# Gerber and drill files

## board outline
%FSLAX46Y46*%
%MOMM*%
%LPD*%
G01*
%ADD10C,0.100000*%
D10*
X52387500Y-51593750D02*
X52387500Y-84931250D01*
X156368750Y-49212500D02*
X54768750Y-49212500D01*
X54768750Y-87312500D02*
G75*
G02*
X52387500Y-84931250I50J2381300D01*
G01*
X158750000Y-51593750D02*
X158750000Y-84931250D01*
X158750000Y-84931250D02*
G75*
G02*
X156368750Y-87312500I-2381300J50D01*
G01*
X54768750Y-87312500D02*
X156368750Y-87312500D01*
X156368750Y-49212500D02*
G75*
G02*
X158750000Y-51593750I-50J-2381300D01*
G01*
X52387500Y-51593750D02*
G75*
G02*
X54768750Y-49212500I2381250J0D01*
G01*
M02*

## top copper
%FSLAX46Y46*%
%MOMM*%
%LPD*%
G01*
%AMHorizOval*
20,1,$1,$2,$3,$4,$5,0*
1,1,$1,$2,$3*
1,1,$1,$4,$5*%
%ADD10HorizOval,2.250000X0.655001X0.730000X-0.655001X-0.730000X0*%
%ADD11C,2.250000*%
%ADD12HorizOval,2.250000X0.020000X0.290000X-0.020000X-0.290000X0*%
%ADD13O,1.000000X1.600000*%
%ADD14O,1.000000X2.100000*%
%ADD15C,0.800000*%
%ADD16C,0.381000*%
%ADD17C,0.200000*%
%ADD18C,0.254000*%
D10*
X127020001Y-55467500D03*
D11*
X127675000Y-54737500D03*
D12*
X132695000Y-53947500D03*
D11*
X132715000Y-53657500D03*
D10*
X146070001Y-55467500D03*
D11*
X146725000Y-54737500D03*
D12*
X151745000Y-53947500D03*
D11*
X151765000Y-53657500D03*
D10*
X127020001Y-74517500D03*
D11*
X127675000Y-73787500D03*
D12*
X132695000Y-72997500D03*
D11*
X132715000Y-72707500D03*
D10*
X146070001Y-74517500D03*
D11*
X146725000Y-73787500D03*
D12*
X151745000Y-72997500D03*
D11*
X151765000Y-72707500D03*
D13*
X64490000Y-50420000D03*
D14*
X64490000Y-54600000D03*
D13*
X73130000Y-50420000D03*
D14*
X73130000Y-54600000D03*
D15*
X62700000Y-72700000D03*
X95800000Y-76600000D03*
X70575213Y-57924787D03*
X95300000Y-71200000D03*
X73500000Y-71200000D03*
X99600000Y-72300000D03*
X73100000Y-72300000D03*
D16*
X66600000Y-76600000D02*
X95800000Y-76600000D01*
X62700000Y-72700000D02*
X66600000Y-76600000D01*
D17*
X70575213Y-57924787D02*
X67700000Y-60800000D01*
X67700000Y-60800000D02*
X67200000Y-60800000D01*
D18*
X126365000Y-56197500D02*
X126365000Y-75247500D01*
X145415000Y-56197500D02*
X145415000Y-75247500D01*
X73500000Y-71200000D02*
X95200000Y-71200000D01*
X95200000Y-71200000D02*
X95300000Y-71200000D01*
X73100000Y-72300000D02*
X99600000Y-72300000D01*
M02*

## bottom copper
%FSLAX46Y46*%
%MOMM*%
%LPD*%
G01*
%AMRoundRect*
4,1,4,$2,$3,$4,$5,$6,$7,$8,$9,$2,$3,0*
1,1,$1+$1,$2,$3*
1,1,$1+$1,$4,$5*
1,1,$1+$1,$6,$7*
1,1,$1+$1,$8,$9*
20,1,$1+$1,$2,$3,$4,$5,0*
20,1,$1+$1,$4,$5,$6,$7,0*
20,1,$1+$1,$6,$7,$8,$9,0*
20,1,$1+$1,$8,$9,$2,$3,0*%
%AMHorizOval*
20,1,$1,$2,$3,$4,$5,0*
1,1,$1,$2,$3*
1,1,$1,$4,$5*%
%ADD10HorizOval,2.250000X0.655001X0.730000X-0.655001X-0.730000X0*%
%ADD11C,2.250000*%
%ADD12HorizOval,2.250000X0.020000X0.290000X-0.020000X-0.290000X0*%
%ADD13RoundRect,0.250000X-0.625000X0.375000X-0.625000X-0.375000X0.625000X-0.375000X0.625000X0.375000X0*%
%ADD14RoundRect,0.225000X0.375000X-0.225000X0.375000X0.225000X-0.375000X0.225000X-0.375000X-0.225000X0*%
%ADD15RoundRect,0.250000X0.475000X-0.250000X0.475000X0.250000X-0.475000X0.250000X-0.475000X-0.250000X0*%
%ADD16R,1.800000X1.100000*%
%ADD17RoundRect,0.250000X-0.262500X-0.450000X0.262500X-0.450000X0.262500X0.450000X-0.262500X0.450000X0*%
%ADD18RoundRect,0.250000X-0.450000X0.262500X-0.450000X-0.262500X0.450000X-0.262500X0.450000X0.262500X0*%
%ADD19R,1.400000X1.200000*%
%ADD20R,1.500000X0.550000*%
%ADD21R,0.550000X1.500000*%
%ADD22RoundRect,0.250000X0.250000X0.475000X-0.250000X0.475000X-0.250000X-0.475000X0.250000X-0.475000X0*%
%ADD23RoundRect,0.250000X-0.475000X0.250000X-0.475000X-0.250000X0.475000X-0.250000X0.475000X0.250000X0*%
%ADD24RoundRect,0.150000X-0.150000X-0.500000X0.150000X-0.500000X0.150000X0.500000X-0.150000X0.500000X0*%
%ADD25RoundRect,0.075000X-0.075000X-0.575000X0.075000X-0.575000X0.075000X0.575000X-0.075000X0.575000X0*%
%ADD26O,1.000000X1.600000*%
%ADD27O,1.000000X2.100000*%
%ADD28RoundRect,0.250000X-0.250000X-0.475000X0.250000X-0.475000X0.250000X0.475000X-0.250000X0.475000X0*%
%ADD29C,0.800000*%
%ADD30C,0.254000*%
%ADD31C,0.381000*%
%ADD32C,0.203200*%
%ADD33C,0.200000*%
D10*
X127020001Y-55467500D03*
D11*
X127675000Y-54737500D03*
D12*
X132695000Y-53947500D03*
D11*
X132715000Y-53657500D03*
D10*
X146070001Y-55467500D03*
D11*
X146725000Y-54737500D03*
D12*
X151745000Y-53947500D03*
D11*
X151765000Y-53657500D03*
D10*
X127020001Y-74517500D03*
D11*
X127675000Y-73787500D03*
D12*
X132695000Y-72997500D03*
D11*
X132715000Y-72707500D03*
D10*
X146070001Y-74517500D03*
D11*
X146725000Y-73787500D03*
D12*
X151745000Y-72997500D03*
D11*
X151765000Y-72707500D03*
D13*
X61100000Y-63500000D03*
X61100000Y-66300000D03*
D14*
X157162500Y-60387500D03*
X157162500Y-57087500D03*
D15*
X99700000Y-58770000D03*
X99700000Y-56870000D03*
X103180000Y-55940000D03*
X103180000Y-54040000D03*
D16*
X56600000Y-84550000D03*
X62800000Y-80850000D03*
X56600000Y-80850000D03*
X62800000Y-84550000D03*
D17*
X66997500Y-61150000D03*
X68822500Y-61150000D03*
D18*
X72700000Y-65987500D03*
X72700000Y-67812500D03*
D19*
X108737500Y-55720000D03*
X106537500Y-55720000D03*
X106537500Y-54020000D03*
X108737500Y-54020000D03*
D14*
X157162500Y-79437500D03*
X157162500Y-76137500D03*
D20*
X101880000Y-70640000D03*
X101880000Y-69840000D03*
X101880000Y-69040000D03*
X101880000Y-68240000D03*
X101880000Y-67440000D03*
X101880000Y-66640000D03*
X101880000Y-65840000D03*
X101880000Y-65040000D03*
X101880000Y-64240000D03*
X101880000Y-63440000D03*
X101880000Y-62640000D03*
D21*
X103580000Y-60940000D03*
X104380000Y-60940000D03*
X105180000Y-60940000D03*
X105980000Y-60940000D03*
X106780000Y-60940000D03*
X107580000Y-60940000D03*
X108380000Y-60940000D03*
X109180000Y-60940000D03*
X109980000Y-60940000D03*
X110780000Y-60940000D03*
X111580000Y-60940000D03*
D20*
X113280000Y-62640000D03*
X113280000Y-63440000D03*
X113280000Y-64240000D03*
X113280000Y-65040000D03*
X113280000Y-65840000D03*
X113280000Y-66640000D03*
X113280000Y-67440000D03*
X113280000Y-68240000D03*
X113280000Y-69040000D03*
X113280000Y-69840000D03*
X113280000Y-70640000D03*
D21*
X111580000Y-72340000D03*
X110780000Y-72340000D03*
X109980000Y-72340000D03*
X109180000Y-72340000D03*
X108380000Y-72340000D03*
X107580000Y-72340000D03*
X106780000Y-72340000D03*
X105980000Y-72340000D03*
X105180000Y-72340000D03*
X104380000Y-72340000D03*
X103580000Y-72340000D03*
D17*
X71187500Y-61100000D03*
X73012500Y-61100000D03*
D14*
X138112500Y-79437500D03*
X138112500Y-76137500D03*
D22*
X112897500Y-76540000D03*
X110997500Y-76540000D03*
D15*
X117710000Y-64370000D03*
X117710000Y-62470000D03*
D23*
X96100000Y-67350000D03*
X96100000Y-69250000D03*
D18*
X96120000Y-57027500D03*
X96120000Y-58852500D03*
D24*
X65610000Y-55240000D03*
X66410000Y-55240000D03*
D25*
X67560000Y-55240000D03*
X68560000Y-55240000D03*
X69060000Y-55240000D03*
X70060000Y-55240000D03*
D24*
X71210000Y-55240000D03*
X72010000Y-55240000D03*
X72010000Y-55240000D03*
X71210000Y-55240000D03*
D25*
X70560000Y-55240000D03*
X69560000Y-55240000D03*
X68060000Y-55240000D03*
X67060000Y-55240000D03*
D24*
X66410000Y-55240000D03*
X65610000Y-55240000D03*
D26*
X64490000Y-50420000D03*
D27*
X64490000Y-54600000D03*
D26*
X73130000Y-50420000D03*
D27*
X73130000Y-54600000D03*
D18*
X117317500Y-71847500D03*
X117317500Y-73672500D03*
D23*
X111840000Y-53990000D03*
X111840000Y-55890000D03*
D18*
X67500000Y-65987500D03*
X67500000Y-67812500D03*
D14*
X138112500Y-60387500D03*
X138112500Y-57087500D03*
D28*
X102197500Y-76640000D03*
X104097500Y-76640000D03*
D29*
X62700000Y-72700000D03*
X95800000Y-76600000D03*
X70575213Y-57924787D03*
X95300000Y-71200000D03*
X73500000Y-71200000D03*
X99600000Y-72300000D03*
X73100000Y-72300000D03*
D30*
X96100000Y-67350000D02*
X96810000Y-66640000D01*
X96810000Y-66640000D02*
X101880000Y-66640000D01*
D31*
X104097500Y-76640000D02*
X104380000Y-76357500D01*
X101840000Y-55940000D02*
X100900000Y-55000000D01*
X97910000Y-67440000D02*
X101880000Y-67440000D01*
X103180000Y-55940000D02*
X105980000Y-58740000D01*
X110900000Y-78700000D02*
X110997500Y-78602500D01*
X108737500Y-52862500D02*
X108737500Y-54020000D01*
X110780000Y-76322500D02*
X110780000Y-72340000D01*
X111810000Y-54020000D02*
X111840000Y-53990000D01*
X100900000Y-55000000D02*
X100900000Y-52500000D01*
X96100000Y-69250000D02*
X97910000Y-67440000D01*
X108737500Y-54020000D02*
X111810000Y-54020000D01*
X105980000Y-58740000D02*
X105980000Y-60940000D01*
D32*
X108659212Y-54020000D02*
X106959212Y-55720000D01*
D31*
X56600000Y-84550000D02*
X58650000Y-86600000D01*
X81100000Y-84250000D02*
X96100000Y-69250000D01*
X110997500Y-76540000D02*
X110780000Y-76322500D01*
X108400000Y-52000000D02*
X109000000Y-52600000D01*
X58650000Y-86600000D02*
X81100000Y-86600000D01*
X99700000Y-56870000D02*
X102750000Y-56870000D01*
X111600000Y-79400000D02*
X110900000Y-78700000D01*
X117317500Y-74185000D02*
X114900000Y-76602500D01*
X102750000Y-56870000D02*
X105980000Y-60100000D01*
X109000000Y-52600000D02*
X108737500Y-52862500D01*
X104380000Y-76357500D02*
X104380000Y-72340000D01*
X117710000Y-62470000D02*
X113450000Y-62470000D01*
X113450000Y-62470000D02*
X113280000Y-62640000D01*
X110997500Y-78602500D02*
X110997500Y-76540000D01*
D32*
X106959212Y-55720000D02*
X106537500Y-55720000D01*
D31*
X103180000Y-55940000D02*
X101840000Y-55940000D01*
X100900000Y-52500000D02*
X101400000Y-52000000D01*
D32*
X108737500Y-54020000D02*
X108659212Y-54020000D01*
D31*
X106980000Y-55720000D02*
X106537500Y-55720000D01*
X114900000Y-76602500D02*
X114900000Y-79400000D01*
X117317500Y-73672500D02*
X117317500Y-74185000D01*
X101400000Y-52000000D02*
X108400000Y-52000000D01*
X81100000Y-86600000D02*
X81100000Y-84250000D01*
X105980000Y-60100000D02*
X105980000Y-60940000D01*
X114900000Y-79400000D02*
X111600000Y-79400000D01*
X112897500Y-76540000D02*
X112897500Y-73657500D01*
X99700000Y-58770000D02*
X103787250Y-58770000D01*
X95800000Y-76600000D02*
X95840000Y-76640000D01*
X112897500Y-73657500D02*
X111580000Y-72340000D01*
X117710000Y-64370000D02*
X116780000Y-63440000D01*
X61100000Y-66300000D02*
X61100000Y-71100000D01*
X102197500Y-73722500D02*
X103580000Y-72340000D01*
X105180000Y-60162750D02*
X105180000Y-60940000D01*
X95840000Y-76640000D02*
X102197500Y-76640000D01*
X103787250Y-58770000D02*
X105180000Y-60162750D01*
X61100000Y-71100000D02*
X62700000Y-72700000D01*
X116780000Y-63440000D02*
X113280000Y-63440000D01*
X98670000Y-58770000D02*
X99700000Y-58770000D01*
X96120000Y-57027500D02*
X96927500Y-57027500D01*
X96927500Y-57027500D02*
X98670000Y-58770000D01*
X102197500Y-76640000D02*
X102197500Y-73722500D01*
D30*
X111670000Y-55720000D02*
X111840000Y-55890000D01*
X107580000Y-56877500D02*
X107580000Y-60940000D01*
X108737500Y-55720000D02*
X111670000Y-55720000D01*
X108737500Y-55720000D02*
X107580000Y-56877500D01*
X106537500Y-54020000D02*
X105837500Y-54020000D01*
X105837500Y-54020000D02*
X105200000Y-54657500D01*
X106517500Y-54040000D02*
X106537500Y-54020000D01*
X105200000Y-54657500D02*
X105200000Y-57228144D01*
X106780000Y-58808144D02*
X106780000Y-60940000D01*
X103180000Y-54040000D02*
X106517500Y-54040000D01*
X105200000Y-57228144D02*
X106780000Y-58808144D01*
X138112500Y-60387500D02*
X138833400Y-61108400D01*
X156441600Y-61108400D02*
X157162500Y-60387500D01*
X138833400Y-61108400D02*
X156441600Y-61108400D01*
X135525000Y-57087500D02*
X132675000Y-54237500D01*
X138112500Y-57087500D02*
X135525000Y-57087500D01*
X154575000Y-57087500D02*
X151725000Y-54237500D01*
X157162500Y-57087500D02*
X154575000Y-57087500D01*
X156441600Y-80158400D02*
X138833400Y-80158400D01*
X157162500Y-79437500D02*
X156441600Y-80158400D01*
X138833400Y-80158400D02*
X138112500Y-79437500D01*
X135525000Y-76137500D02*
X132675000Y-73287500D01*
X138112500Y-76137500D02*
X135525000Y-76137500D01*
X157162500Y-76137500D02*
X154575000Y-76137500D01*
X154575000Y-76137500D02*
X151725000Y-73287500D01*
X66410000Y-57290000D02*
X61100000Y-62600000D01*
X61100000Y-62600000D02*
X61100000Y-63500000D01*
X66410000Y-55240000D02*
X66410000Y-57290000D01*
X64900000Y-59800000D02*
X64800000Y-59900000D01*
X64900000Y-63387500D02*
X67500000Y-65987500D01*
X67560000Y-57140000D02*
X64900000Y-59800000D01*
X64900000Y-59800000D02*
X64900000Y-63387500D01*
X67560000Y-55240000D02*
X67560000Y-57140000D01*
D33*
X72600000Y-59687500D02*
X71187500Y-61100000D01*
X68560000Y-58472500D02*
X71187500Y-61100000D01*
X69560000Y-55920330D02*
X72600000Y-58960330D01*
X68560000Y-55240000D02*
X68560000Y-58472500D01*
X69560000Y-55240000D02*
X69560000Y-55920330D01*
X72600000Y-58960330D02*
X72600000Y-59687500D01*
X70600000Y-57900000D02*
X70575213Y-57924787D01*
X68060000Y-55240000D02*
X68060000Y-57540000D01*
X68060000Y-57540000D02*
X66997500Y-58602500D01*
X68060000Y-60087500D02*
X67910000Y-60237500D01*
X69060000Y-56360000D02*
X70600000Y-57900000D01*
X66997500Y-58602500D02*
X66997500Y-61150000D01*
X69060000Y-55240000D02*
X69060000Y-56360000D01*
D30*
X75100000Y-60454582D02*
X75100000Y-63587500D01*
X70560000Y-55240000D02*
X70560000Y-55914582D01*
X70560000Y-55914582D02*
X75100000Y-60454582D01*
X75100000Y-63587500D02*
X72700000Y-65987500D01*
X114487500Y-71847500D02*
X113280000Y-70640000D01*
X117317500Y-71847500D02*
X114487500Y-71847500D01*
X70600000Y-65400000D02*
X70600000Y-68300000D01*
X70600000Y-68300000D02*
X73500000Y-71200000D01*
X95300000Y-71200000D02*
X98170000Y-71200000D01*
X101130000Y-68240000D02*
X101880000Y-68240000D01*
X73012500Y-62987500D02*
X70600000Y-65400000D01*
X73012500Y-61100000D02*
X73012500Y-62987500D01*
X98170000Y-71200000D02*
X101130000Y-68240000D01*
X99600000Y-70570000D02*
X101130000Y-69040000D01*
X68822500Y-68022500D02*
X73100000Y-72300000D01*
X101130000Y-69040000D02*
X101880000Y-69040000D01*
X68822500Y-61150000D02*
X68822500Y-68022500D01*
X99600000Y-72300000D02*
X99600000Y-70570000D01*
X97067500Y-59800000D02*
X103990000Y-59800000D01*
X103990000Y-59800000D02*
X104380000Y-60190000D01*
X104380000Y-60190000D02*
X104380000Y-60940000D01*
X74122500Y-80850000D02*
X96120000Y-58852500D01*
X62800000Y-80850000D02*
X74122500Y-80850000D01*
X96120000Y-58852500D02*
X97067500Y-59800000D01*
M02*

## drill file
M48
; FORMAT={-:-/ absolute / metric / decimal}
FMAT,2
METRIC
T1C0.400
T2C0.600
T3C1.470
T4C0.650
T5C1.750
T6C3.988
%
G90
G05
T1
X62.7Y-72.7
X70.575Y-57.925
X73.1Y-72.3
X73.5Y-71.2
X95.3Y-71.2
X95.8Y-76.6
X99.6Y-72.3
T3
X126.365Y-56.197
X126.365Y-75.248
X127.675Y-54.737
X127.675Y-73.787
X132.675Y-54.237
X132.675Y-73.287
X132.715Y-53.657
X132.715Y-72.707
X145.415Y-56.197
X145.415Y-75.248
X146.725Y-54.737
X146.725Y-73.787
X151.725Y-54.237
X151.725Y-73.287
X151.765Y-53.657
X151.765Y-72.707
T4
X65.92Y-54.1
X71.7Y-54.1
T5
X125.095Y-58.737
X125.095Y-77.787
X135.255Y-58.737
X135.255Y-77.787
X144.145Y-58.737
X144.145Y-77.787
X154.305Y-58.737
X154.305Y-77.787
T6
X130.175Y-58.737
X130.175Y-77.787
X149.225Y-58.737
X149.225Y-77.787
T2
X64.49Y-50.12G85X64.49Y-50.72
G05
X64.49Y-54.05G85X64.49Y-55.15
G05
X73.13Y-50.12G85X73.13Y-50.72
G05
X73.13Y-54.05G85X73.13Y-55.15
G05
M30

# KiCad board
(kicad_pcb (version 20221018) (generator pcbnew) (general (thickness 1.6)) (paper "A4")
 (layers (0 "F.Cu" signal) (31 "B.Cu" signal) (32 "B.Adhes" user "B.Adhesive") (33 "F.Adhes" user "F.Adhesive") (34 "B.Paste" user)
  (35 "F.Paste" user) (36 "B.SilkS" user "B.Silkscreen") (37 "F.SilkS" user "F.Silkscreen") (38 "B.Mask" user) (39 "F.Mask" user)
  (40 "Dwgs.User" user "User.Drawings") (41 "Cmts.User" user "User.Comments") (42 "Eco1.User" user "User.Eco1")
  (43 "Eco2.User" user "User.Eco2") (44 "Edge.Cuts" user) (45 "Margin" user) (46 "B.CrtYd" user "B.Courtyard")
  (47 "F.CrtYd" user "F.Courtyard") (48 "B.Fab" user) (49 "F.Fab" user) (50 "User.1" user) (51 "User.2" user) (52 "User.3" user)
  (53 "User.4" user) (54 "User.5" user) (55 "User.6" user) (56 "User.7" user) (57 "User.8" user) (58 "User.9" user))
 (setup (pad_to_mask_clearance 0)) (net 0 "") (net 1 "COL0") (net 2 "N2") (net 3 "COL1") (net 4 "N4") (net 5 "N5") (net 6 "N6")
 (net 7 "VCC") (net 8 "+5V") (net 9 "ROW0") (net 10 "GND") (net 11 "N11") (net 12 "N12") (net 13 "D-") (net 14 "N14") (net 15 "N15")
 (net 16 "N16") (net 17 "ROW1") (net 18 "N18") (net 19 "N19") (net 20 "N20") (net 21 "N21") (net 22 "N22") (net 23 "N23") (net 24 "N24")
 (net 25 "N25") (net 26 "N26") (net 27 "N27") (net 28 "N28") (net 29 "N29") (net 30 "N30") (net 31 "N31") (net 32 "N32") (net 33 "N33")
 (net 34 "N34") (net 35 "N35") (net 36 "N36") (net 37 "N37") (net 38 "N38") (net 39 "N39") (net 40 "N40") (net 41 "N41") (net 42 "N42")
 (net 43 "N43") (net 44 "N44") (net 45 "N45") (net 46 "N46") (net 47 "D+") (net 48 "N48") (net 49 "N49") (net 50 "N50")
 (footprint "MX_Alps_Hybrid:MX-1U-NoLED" (layer "F.Cu") (at 130.175 58.7375)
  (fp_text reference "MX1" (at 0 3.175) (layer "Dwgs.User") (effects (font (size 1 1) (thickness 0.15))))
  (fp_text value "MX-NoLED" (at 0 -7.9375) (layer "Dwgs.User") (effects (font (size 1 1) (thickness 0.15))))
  (pad "" np_thru_hole circle (at -5.08 0 48.0996) (size 1.75 1.75) (drill 1.75) (layers "*.Cu" "*.Mask"))
  (pad "" np_thru_hole circle (at 0 0) (size 3.9878 3.9878) (drill 3.9878) (layers "*.Cu" "*.Mask"))
  (pad "" np_thru_hole circle (at 5.08 0 48.0996) (size 1.75 1.75) (drill 1.75) (layers "*.Cu" "*.Mask"))
  (pad "1" thru_hole oval (at -3.81 -2.54 48.0996) (size 4.211556 2.25) (drill 1.47 (offset 0.980778 0)) (layers "*.Cu" "B.Mask")
   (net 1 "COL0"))
  (pad "1" thru_hole circle (at -2.5 -4) (size 2.25 2.25) (drill 1.47) (layers "*.Cu" "B.Mask") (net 1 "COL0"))
  (pad "2" thru_hole oval (at 2.5 -4.5 86.0548) (size 2.831378 2.25) (drill 1.47 (offset 0.290689 0)) (layers "*.Cu" "B.Mask") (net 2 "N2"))
  (pad "2" thru_hole circle (at 2.54 -5.08) (size 2.25 2.25) (drill 1.47) (layers "*.Cu" "B.Mask") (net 2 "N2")))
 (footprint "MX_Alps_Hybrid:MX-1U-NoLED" (layer "F.Cu") (at 149.225 58.7375)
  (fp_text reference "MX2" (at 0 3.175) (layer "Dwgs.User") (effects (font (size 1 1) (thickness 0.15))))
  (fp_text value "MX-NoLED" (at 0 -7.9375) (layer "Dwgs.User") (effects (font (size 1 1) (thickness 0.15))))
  (pad "" np_thru_hole circle (at -5.08 0 48.0996) (size 1.75 1.75) (drill 1.75) (layers "*.Cu" "*.Mask"))
  (pad "" np_thru_hole circle (at 0 0) (size 3.9878 3.9878) (drill 3.9878) (layers "*.Cu" "*.Mask"))
  (pad "" np_thru_hole circle (at 5.08 0 48.0996) (size 1.75 1.75) (drill 1.75) (layers "*.Cu" "*.Mask"))
  (pad "1" thru_hole oval (at -3.81 -2.54 48.0996) (size 4.211556 2.25) (drill 1.47 (offset 0.980778 0)) (layers "*.Cu" "B.Mask")
   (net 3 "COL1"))
  (pad "1" thru_hole circle (at -2.5 -4) (size 2.25 2.25) (drill 1.47) (layers "*.Cu" "B.Mask") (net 3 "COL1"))
  (pad "2" thru_hole oval (at 2.5 -4.5 86.0548) (size 2.831378 2.25) (drill 1.47 (offset 0.290689 0)) (layers "*.Cu" "B.Mask") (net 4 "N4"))
  (pad "2" thru_hole circle (at 2.54 -5.08) (size 2.25 2.25) (drill 1.47) (layers "*.Cu" "B.Mask") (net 4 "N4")))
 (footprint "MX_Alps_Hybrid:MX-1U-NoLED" (layer "F.Cu") (at 130.175 77.7875)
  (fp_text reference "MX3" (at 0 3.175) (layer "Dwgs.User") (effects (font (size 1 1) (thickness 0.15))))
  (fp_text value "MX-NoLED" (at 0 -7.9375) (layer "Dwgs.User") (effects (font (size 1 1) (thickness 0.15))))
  (pad "" np_thru_hole circle (at -5.08 0 48.0996) (size 1.75 1.75) (drill 1.75) (layers "*.Cu" "*.Mask"))
  (pad "" np_thru_hole circle (at 0 0) (size 3.9878 3.9878) (drill 3.9878) (layers "*.Cu" "*.Mask"))
  (pad "" np_thru_hole circle (at 5.08 0 48.0996) (size 1.75 1.75) (drill 1.75) (layers "*.Cu" "*.Mask"))
  (pad "1" thru_hole oval (at -3.81 -2.54 48.0996) (size 4.211556 2.25) (drill 1.47 (offset 0.980778 0)) (layers "*.Cu" "B.Mask")
   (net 1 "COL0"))
  (pad "1" thru_hole circle (at -2.5 -4) (size 2.25 2.25) (drill 1.47) (layers "*.Cu" "B.Mask") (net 1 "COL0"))
  (pad "2" thru_hole oval (at 2.5 -4.5 86.0548) (size 2.831378 2.25) (drill 1.47 (offset 0.290689 0)) (layers "*.Cu" "B.Mask") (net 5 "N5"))
  (pad "2" thru_hole circle (at 2.54 -5.08) (size 2.25 2.25) (drill 1.47) (layers "*.Cu" "B.Mask") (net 5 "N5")))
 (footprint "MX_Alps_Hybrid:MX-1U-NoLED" (layer "F.Cu") (at 149.225 77.7875)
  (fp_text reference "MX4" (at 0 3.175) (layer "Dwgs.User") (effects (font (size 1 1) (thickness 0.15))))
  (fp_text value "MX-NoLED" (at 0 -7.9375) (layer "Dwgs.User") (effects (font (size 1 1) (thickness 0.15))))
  (pad "" np_thru_hole circle (at -5.08 0 48.0996) (size 1.75 1.75) (drill 1.75) (layers "*.Cu" "*.Mask"))
  (pad "" np_thru_hole circle (at 0 0) (size 3.9878 3.9878) (drill 3.9878) (layers "*.Cu" "*.Mask"))
  (pad "" np_thru_hole circle (at 5.08 0 48.0996) (size 1.75 1.75) (drill 1.75) (layers "*.Cu" "*.Mask"))
  (pad "1" thru_hole oval (at -3.81 -2.54 48.0996) (size 4.211556 2.25) (drill 1.47 (offset 0.980778 0)) (layers "*.Cu" "B.Mask")
   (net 3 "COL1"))
  (pad "1" thru_hole circle (at -2.5 -4) (size 2.25 2.25) (drill 1.47) (layers "*.Cu" "B.Mask") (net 3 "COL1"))
  (pad "2" thru_hole oval (at 2.5 -4.5 86.0548) (size 2.831378 2.25) (drill 1.47 (offset 0.290689 0)) (layers "*.Cu" "B.Mask") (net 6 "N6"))
  (pad "2" thru_hole circle (at 2.54 -5.08) (size 2.25 2.25) (drill 1.47) (layers "*.Cu" "B.Mask") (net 6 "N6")))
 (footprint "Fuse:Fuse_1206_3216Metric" (layer "B.Cu") (at 61.1 64.9 -90)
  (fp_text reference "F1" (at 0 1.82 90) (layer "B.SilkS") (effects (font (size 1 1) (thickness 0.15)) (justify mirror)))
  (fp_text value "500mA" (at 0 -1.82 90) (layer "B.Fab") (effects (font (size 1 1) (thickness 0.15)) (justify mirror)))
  (pad "1" smd roundrect (at -1.4 0 270) (size 1.25 1.75) (layers "B.Cu" "B.Paste" "B.Mask") (roundrect_rratio 0.2) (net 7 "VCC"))
  (pad "2" smd roundrect (at 1.4 0 270) (size 1.25 1.75) (layers "B.Cu" "B.Paste" "B.Mask") (roundrect_rratio 0.2) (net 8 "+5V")))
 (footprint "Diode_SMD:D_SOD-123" (layer "B.Cu") (at 157.1625 58.7375 90)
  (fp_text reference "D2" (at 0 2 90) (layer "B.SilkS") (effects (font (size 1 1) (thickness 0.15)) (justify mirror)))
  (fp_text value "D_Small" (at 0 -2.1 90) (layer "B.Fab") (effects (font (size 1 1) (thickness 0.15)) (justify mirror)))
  (pad "1" smd roundrect (at -1.65 0 90) (size 0.9 1.2) (layers "B.Cu" "B.Paste" "B.Mask") (roundrect_rratio 0.25) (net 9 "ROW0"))
  (pad "2" smd roundrect (at 1.65 0 90) (size 0.9 1.2) (layers "B.Cu" "B.Paste" "B.Mask") (roundrect_rratio 0.25) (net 4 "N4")))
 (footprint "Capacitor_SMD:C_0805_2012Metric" (layer "B.Cu") (at 99.7 57.82 90)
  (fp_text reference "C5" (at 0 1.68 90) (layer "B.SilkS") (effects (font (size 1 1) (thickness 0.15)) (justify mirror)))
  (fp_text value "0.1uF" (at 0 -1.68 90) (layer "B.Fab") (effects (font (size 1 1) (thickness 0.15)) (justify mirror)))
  (pad "1" smd roundrect (at -0.95 0 90) (size 1 1.45) (layers "B.Cu" "B.Paste" "B.Mask") (roundrect_rratio 0.25) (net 8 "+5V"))
  (pad "2" smd roundrect (at 0.95 0 90) (size 1 1.45) (layers "B.Cu" "B.Paste" "B.Mask") (roundrect_rratio 0.25) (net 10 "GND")))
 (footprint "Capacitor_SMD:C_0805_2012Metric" (layer "B.Cu") (at 103.18 54.99 90)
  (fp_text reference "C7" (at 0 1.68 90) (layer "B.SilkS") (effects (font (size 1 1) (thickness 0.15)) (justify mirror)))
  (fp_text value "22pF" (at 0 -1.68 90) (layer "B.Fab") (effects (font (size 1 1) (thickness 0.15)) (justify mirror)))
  (pad "1" smd roundrect (at -0.95 0 90) (size 1 1.45) (layers "B.Cu" "B.Paste" "B.Mask") (roundrect_rratio 0.25) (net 10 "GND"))
  (pad "2" smd roundrect (at 0.95 0 90) (size 1 1.45) (layers "B.Cu" "B.Paste" "B.Mask") (roundrect_rratio 0.25) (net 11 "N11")))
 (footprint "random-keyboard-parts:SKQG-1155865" (layer "B.Cu") (at 59.7 82.7 180)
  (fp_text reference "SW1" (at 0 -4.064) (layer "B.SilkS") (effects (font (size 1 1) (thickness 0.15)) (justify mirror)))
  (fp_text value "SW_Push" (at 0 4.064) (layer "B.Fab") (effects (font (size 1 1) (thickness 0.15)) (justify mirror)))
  (pad "1" smd rect (at 3.1 -1.85 180) (size 1.8 1.1) (layers "B.Cu" "B.Paste" "B.Mask") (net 10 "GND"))
  (pad "2" smd rect (at -3.1 1.85 180) (size 1.8 1.1) (layers "B.Cu" "B.Paste" "B.Mask") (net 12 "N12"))
  (pad "3" smd rect (at 3.1 1.85 180) (size 1.8 1.1) (layers "B.Cu" "B.Paste" "B.Mask"))
  (pad "4" smd rect (at -3.1 -1.85 180) (size 1.8 1.1) (layers "B.Cu" "B.Paste" "B.Mask")))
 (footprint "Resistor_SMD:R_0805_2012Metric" (layer "B.Cu") (at 67.91 61.15)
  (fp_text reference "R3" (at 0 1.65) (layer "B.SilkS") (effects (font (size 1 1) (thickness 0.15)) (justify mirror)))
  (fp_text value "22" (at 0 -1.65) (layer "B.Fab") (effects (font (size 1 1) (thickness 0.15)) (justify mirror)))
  (pad "1" smd roundrect (at -0.9125 0) (size 1.025 1.4) (layers "B.Cu" "B.Paste" "B.Mask") (roundrect_rratio 0.243902) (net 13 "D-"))
  (pad "2" smd roundrect (at 0.9125 0) (size 1.025 1.4) (layers "B.Cu" "B.Paste" "B.Mask") (roundrect_rratio 0.243902) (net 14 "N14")))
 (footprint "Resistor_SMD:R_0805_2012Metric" (layer "B.Cu") (at 72.7 66.9 -90)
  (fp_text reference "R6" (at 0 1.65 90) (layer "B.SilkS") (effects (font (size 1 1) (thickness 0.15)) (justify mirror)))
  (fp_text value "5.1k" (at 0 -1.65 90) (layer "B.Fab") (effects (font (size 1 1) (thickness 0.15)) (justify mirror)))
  (pad "1" smd roundrect (at -0.9125 0 270) (size 1.025 1.4) (layers "B.Cu" "B.Paste" "B.Mask") (roundrect_rratio 0.243902) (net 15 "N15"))
  (pad "2" smd roundrect (at 0.9125 0 270) (size 1.025 1.4) (layers "B.Cu" "B.Paste" "B.Mask") (roundrect_rratio 0.243902) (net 10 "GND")))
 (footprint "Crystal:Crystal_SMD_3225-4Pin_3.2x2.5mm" (layer "B.Cu") (at 107.6375 54.87 180)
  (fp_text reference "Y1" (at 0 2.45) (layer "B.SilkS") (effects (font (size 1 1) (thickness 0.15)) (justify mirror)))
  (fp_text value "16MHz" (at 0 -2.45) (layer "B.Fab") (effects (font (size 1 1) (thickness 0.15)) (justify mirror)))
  (pad "1" smd rect (at -1.1 -0.85 180) (size 1.4 1.2) (layers "B.Cu" "B.Paste" "B.Mask") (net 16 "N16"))
  (pad "2" smd rect (at 1.1 -0.85 180) (size 1.4 1.2) (layers "B.Cu" "B.Paste" "B.Mask") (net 10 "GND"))
  (pad "3" smd rect (at 1.1 0.85 180) (size 1.4 1.2) (layers "B.Cu" "B.Paste" "B.Mask") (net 11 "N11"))
  (pad "4" smd rect (at -1.1 0.85 180) (size 1.4 1.2) (layers "B.Cu" "B.Paste" "B.Mask") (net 10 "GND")))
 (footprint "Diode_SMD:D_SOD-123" (layer "B.Cu") (at 157.1625 77.7875 90)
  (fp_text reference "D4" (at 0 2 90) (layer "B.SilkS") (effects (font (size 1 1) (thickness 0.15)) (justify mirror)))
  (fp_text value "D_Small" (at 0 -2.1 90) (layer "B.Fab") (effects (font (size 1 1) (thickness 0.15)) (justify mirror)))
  (pad "1" smd roundrect (at -1.65 0 90) (size 0.9 1.2) (layers "B.Cu" "B.Paste" "B.Mask") (roundrect_rratio 0.25) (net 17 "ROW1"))
  (pad "2" smd roundrect (at 1.65 0 90) (size 0.9 1.2) (layers "B.Cu" "B.Paste" "B.Mask") (roundrect_rratio 0.25) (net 6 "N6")))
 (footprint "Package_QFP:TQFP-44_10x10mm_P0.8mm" (layer "B.Cu") (at 107.58 66.64)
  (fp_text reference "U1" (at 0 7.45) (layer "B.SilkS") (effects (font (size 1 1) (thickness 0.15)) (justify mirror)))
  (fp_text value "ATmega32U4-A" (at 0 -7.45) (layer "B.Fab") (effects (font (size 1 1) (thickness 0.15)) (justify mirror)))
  (pad "1" smd rect (at -5.7 4) (size 1.5 0.55) (layers "B.Cu" "B.Paste" "B.Mask") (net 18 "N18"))
  (pad "2" smd rect (at -5.7 3.2) (size 1.5 0.55) (layers "B.Cu" "B.Paste" "B.Mask") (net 8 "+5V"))
  (pad "3" smd rect (at -5.7 2.4) (size 1.5 0.55) (layers "B.Cu" "B.Paste" "B.Mask") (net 14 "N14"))
  (pad "4" smd rect (at -5.7 1.6) (size 1.5 0.55) (layers "B.Cu" "B.Paste" "B.Mask") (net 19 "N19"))
  (pad "5" smd rect (at -5.7 0.8) (size 1.5 0.55) (layers "B.Cu" "B.Paste" "B.Mask") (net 10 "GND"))
  (pad "6" smd rect (at -5.7 0) (size 1.5 0.55) (layers "B.Cu" "B.Paste" "B.Mask") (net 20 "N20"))
  (pad "7" smd rect (at -5.7 -0.8) (size 1.5 0.55) (layers "B.Cu" "B.Paste" "B.Mask") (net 8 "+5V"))
  (pad "8" smd rect (at -5.7 -1.6) (size 1.5 0.55) (layers "B.Cu" "B.Paste" "B.Mask") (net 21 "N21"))
  (pad "9" smd rect (at -5.7 -2.4) (size 1.5 0.55) (layers "B.Cu" "B.Paste" "B.Mask") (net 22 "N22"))
  (pad "10" smd rect (at -5.7 -3.2) (size 1.5 0.55) (layers "B.Cu" "B.Paste" "B.Mask") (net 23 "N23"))
  (pad "11" smd rect (at -5.7 -4) (size 1.5 0.55) (layers "B.Cu" "B.Paste" "B.Mask") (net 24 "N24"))
  (pad "12" smd rect (at -4 -5.7 270) (size 1.5 0.55) (layers "B.Cu" "B.Paste" "B.Mask") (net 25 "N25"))
  (pad "13" smd rect (at -3.2 -5.7 270) (size 1.5 0.55) (layers "B.Cu" "B.Paste" "B.Mask") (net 12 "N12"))
  (pad "14" smd rect (at -2.4 -5.7 270) (size 1.5 0.55) (layers "B.Cu" "B.Paste" "B.Mask") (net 8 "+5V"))
  (pad "15" smd rect (at -1.6 -5.7 270) (size 1.5 0.55) (layers "B.Cu" "B.Paste" "B.Mask") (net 10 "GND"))
  (pad "16" smd rect (at -0.8 -5.7 270) (size 1.5 0.55) (layers "B.Cu" "B.Paste" "B.Mask") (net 11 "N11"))
  (pad "17" smd rect (at 0 -5.7 270) (size 1.5 0.55) (layers "B.Cu" "B.Paste" "B.Mask") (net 16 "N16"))
  (pad "18" smd rect (at 0.8 -5.7 270) (size 1.5 0.55) (layers "B.Cu" "B.Paste" "B.Mask") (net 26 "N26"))
  (pad "19" smd rect (at 1.6 -5.7 270) (size 1.5 0.55) (layers "B.Cu" "B.Paste" "B.Mask") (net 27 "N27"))
  (pad "20" smd rect (at 2.4 -5.7 270) (size 1.5 0.55) (layers "B.Cu" "B.Paste" "B.Mask") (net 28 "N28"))
  (pad "21" smd rect (at 3.2 -5.7 270) (size 1.5 0.55) (layers "B.Cu" "B.Paste" "B.Mask") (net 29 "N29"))
  (pad "22" smd rect (at 4 -5.7 270) (size 1.5 0.55) (layers "B.Cu" "B.Paste" "B.Mask") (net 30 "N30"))
  (pad "23" smd rect (at 5.7 -4) (size 1.5 0.55) (layers "B.Cu" "B.Paste" "B.Mask") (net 10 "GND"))
  (pad "24" smd rect (at 5.7 -3.2) (size 1.5 0.55) (layers "B.Cu" "B.Paste" "B.Mask") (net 8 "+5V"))
  (pad "25" smd rect (at 5.7 -2.4) (size 1.5 0.55) (layers "B.Cu" "B.Paste" "B.Mask") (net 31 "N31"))
  (pad "26" smd rect (at 5.7 -1.6) (size 1.5 0.55) (layers "B.Cu" "B.Paste" "B.Mask") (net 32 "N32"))
  (pad "27" smd rect (at 5.7 -0.8) (size 1.5 0.55) (layers "B.Cu" "B.Paste" "B.Mask") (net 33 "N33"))
  (pad "28" smd rect (at 5.7 0) (size 1.5 0.55) (layers "B.Cu" "B.Paste" "B.Mask") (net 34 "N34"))
  (pad "29" smd rect (at 5.7 0.8) (size 1.5 0.55) (layers "B.Cu" "B.Paste" "B.Mask") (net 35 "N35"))
  (pad "30" smd rect (at 5.7 1.6) (size 1.5 0.55) (layers "B.Cu" "B.Paste" "B.Mask") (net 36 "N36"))
  (pad "31" smd rect (at 5.7 2.4) (size 1.5 0.55) (layers "B.Cu" "B.Paste" "B.Mask") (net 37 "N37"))
  (pad "32" smd rect (at 5.7 3.2) (size 1.5 0.55) (layers "B.Cu" "B.Paste" "B.Mask") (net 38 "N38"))
  (pad "33" smd rect (at 5.7 4) (size 1.5 0.55) (layers "B.Cu" "B.Paste" "B.Mask") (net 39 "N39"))
  (pad "34" smd rect (at 4 5.7 270) (size 1.5 0.55) (layers "B.Cu" "B.Paste" "B.Mask") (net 8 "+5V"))
  (pad "35" smd rect (at 3.2 5.7 270) (size 1.5 0.55) (layers "B.Cu" "B.Paste" "B.Mask") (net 10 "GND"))
  (pad "36" smd rect (at 2.4 5.7 270) (size 1.5 0.55) (layers "B.Cu" "B.Paste" "B.Mask") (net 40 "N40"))
  (pad "37" smd rect (at 1.6 5.7 270) (size 1.5 0.55) (layers "B.Cu" "B.Paste" "B.Mask") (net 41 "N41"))
  (pad "38" smd rect (at 0.8 5.7 270) (size 1.5 0.55) (layers "B.Cu" "B.Paste" "B.Mask") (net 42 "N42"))
  (pad "39" smd rect (at 0 5.7 270) (size 1.5 0.55) (layers "B.Cu" "B.Paste" "B.Mask") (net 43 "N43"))
  (pad "40" smd rect (at -0.8 5.7 270) (size 1.5 0.55) (layers "B.Cu" "B.Paste" "B.Mask") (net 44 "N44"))
  (pad "41" smd rect (at -1.6 5.7 270) (size 1.5 0.55) (layers "B.Cu" "B.Paste" "B.Mask") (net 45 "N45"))
  (pad "42" smd rect (at -2.4 5.7 270) (size 1.5 0.55) (layers "B.Cu" "B.Paste" "B.Mask") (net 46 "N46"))
  (pad "43" smd rect (at -3.2 5.7 270) (size 1.5 0.55) (layers "B.Cu" "B.Paste" "B.Mask") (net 10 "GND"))
  (pad "44" smd rect (at -4 5.7 270) (size 1.5 0.55) (layers "B.Cu" "B.Paste" "B.Mask") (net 8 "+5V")))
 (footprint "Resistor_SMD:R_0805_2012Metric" (layer "B.Cu") (at 72.1 61.1)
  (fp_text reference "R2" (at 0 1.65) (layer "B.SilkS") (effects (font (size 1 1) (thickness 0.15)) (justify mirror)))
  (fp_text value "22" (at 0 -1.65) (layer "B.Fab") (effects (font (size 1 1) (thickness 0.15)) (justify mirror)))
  (pad "1" smd roundrect (at -0.9125 0) (size 1.025 1.4) (layers "B.Cu" "B.Paste" "B.Mask") (roundrect_rratio 0.243902) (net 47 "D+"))
  (pad "2" smd roundrect (at 0.9125 0) (size 1.025 1.4) (layers "B.Cu" "B.Paste" "B.Mask") (roundrect_rratio 0.243902) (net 19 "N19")))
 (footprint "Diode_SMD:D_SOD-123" (layer "B.Cu") (at 138.1125 77.7875 90)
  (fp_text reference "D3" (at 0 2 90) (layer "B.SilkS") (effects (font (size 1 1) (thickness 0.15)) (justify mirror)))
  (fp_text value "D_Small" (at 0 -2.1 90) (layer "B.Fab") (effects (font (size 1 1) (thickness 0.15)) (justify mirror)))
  (pad "1" smd roundrect (at -1.65 0 90) (size 0.9 1.2) (layers "B.Cu" "B.Paste" "B.Mask") (roundrect_rratio 0.25) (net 17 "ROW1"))
  (pad "2" smd roundrect (at 1.65 0 90) (size 0.9 1.2) (layers "B.Cu" "B.Paste" "B.Mask") (roundrect_rratio 0.25) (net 5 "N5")))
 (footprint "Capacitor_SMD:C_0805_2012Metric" (layer "B.Cu") (at 111.9475 76.54 180)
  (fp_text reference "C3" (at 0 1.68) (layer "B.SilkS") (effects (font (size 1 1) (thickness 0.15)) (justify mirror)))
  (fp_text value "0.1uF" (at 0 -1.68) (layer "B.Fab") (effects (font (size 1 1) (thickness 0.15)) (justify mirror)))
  (pad "1" smd roundrect (at -0.95 0 180) (size 1 1.45) (layers "B.Cu" "B.Paste" "B.Mask") (roundrect_rratio 0.25) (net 8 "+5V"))
  (pad "2" smd roundrect (at 0.95 0 180) (size 1 1.45) (layers "B.Cu" "B.Paste" "B.Mask") (roundrect_rratio 0.25) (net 10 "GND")))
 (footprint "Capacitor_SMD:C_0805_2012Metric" (layer "B.Cu") (at 117.71 63.42 90)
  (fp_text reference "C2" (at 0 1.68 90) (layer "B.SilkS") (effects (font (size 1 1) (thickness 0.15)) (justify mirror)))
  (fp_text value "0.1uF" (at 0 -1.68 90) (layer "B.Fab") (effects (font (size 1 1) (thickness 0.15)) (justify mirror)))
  (pad "1" smd roundrect (at -0.95 0 90) (size 1 1.45) (layers "B.Cu" "B.Paste" "B.Mask") (roundrect_rratio 0.25) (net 8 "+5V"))
  (pad "2" smd roundrect (at 0.95 0 90) (size 1 1.45) (layers "B.Cu" "B.Paste" "B.Mask") (roundrect_rratio 0.25) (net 10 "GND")))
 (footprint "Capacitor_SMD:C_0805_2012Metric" (layer "B.Cu") (at 96.1 68.3 -90)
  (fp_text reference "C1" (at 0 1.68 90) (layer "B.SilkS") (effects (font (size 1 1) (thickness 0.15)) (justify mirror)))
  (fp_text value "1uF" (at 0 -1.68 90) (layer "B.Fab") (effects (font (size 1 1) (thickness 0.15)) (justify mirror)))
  (pad "1" smd roundrect (at -0.95 0 270) (size 1 1.45) (layers "B.Cu" "B.Paste" "B.Mask") (roundrect_rratio 0.25) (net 20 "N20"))
  (pad "2" smd roundrect (at 0.95 0 270) (size 1 1.45) (layers "B.Cu" "B.Paste" "B.Mask") (roundrect_rratio 0.25) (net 10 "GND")))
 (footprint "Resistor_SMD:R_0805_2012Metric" (layer "B.Cu") (at 96.12 57.94 -90)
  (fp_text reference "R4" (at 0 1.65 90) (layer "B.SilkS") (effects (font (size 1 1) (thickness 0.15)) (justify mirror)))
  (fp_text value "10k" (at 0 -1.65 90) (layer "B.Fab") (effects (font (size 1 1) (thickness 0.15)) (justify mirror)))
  (pad "1" smd roundrect (at -0.9125 0 270) (size 1.025 1.4) (layers "B.Cu" "B.Paste" "B.Mask") (roundrect_rratio 0.243902) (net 8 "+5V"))
  (pad "2" smd roundrect (at 0.9125 0 270) (size 1.025 1.4) (layers "B.Cu" "B.Paste" "B.Mask") (roundrect_rratio 0.243902) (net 12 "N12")))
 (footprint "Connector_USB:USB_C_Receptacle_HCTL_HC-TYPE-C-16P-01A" (layer "B.Cu") (at 68.81 51.495)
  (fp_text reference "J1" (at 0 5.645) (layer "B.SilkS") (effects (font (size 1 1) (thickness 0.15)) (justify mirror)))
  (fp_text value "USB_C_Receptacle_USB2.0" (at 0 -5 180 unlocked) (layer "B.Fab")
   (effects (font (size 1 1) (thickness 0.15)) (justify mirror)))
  (pad "" np_thru_hole circle (at -2.89 2.605) (size 0.65 0.65) (drill 0.65) (layers "*.Mask"))
  (pad "" np_thru_hole circle (at 2.89 2.605) (size 0.65 0.65) (drill 0.65) (layers "*.Mask"))
  (pad "A1" smd roundrect (at -3.2 3.745) (size 0.6 1.3) (layers "B.Cu" "B.Paste" "B.Mask") (roundrect_rratio 0.25) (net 10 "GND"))
  (pad "A4" smd roundrect (at -2.4 3.745) (size 0.6 1.3) (layers "B.Cu" "B.Paste" "B.Mask") (roundrect_rratio 0.25) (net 7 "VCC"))
  (pad "A5" smd roundrect (at -1.25 3.745) (size 0.3 1.3) (layers "B.Cu" "B.Paste" "B.Mask") (roundrect_rratio 0.25) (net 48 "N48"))
  (pad "A6" smd roundrect (at -0.25 3.745) (size 0.3 1.3) (layers "B.Cu" "B.Paste" "B.Mask") (roundrect_rratio 0.25) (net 47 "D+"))
  (pad "A7" smd roundrect (at 0.25 3.745) (size 0.3 1.3) (layers "B.Cu" "B.Paste" "B.Mask") (roundrect_rratio 0.25) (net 13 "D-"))
  (pad "A8" smd roundrect (at 1.25 3.745) (size 0.3 1.3) (layers "B.Cu" "B.Paste" "B.Mask") (roundrect_rratio 0.25) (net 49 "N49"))
  (pad "A9" smd roundrect (at 2.4 3.745) (size 0.6 1.3) (layers "B.Cu" "B.Paste" "B.Mask") (roundrect_rratio 0.25) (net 7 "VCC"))
  (pad "A12" smd roundrect (at 3.2 3.745) (size 0.6 1.3) (layers "B.Cu" "B.Paste" "B.Mask") (roundrect_rratio 0.25) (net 10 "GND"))
  (pad "B1" smd roundrect (at 3.2 3.745) (size 0.6 1.3) (layers "B.Cu" "B.Paste" "B.Mask") (roundrect_rratio 0.25) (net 10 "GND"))
  (pad "B4" smd roundrect (at 2.4 3.745) (size 0.6 1.3) (layers "B.Cu" "B.Paste" "B.Mask") (roundrect_rratio 0.25) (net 7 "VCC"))
  (pad "B5" smd roundrect (at 1.75 3.745) (size 0.3 1.3) (layers "B.Cu" "B.Paste" "B.Mask") (roundrect_rratio 0.25) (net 15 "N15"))
  (pad "B6" smd roundrect (at 0.75 3.745) (size 0.3 1.3) (layers "B.Cu" "B.Paste" "B.Mask") (roundrect_rratio 0.25) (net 47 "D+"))
  (pad "B7" smd roundrect (at -0.75 3.745) (size 0.3 1.3) (layers "B.Cu" "B.Paste" "B.Mask") (roundrect_rratio 0.25) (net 13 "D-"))
  (pad "B8" smd roundrect (at -1.75 3.745) (size 0.3 1.3) (layers "B.Cu" "B.Paste" "B.Mask") (roundrect_rratio 0.25) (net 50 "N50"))
  (pad "B9" smd roundrect (at -2.4 3.745) (size 0.6 1.3) (layers "B.Cu" "B.Paste" "B.Mask") (roundrect_rratio 0.25) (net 7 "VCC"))
  (pad "B12" smd roundrect (at -3.2 3.745) (size 0.6 1.3) (layers "B.Cu" "B.Paste" "B.Mask") (roundrect_rratio 0.25) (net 10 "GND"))
  (pad "S1" thru_hole oval (at -4.32 -1.075) (size 1 1.6) (drill oval 0.6 1.2) (layers "*.Cu" "*.Mask") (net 10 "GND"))
  (pad "S1" thru_hole oval (at -4.32 3.105) (size 1 2.1) (drill oval 0.6 1.7) (layers "*.Cu" "*.Mask") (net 10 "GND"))
  (pad "S1" thru_hole oval (at 4.32 -1.075) (size 1 1.6) (drill oval 0.6 1.2) (layers "*.Cu" "*.Mask") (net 10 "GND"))
  (pad "S1" thru_hole oval (at 4.32 3.105) (size 1 2.1) (drill oval 0.6 1.7) (layers "*.Cu" "*.Mask") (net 10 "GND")))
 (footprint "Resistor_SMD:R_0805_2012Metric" (layer "B.Cu") (at 117.3175 72.76 -90)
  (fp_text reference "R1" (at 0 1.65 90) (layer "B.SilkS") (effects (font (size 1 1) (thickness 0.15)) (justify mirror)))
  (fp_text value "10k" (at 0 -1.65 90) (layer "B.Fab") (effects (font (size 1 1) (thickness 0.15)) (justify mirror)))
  (pad "1" smd roundrect (at -0.9125 0 270) (size 1.025 1.4) (layers "B.Cu" "B.Paste" "B.Mask") (roundrect_rratio 0.243902) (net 39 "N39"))
  (pad "2" smd roundrect (at 0.9125 0 270) (size 1.025 1.4) (layers "B.Cu" "B.Paste" "B.Mask") (roundrect_rratio 0.243902) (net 10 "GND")))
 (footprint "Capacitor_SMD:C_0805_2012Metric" (layer "B.Cu") (at 111.84 54.94 -90)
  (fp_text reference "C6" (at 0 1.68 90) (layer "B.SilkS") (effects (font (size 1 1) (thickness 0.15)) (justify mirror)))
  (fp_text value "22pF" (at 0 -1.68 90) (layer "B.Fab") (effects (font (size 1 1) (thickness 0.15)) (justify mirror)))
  (pad "1" smd roundrect (at -0.95 0 270) (size 1 1.45) (layers "B.Cu" "B.Paste" "B.Mask") (roundrect_rratio 0.25) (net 10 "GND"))
  (pad "2" smd roundrect (at 0.95 0 270) (size 1 1.45) (layers "B.Cu" "B.Paste" "B.Mask") (roundrect_rratio 0.25) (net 16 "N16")))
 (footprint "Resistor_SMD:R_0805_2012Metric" (layer "B.Cu") (at 67.5 66.9 -90)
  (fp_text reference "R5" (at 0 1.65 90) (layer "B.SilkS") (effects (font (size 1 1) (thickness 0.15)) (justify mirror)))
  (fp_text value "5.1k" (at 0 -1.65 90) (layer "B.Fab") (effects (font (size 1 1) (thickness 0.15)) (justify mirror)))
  (pad "1" smd roundrect (at -0.9125 0 270) (size 1.025 1.4) (layers "B.Cu" "B.Paste" "B.Mask") (roundrect_rratio 0.243902) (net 48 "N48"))
  (pad "2" smd roundrect (at 0.9125 0 270) (size 1.025 1.4) (layers "B.Cu" "B.Paste" "B.Mask") (roundrect_rratio 0.243902) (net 10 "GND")))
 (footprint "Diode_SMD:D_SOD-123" (layer "B.Cu") (at 138.1125 58.7375 90)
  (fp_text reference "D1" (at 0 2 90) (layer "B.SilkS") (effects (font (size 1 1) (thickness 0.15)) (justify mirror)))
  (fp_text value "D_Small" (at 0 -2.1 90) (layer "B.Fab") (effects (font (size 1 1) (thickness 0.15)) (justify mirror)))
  (pad "1" smd roundrect (at -1.65 0 90) (size 0.9 1.2) (layers "B.Cu" "B.Paste" "B.Mask") (roundrect_rratio 0.25) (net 9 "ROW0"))
  (pad "2" smd roundrect (at 1.65 0 90) (size 0.9 1.2) (layers "B.Cu" "B.Paste" "B.Mask") (roundrect_rratio 0.25) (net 2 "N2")))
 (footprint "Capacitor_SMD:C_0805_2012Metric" (layer "B.Cu") (at 103.1475 76.64)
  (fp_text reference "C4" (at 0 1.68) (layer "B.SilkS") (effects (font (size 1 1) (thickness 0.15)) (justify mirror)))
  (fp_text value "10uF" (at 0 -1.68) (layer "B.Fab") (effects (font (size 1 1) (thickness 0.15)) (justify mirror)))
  (pad "1" smd roundrect (at -0.95 0) (size 1 1.45) (layers "B.Cu" "B.Paste" "B.Mask") (roundrect_rratio 0.25) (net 8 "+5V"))
  (pad "2" smd roundrect (at 0.95 0) (size 1 1.45) (layers "B.Cu" "B.Paste" "B.Mask") (roundrect_rratio 0.25) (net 10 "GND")))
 (gr_line (start 52.3875 51.59375) (end 52.3875 84.93125) (stroke (width 0.1) (type default)) (layer "Edge.Cuts"))
 (gr_line (start 156.36875 49.2125) (end 54.76875 49.2125) (stroke (width 0.1) (type default)) (layer "Edge.Cuts"))
 (gr_arc (start 54.76875 87.3125) (mid 53.084952 86.615048) (end 52.3875 84.93125) (stroke (width 0.1) (type default)) (layer "Edge.Cuts"))
 (gr_line (start 158.75 51.59375) (end 158.75 84.93125) (stroke (width 0.1) (type default)) (layer "Edge.Cuts"))
 (gr_arc (start 158.75 84.93125) (mid 158.052548 86.615048) (end 156.36875 87.3125) (stroke (width 0.1) (type default)) (layer "Edge.Cuts"))
 (gr_line (start 54.76875 87.3125) (end 156.36875 87.3125) (stroke (width 0.1) (type default)) (layer "Edge.Cuts"))
 (gr_arc (start 156.36875 49.2125) (mid 158.052548 49.909952) (end 158.75 51.59375) (stroke (width 0.1) (type default)) (layer "Edge.Cuts"))
 (gr_arc (start 52.3875 51.59375) (mid 53.084952 49.909952) (end 54.76875 49.2125) (stroke (width 0.1) (type default)) (layer "Edge.Cuts"))
 (segment (start 96.1 67.35) (end 96.81 66.64) (width 0.254) (layer "B.Cu") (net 20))
 (segment (start 96.81 66.64) (end 101.88 66.64) (width 0.254) (layer "B.Cu") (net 20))
 (segment (start 104.0975 76.64) (end 104.38 76.3575) (width 0.381) (layer "B.Cu") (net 10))
 (segment (start 101.84 55.94) (end 100.9 55) (width 0.381) (layer "B.Cu") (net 10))
 (segment (start 97.91 67.44) (end 101.88 67.44) (width 0.381) (layer "B.Cu") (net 10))
 (segment (start 103.18 55.94) (end 105.98 58.74) (width 0.381) (layer "B.Cu") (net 10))
 (segment (start 110.9 78.7) (end 110.9975 78.6025) (width 0.381) (layer "B.Cu") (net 10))
 (segment (start 108.7375 52.8625) (end 108.7375 54.02) (width 0.381) (layer "B.Cu") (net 10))
 (segment (start 110.78 76.3225) (end 110.78 72.34) (width 0.381) (layer "B.Cu") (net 10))
 (segment (start 111.81 54.02) (end 111.84 53.99) (width 0.381) (layer "B.Cu") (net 10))
 (segment (start 100.9 55) (end 100.9 52.5) (width 0.381) (layer "B.Cu") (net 10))
 (segment (start 96.1 69.25) (end 97.91 67.44) (width 0.381) (layer "B.Cu") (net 10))
 (segment (start 108.7375 54.02) (end 111.81 54.02) (width 0.381) (layer "B.Cu") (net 10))
 (segment (start 105.98 58.74) (end 105.98 60.94) (width 0.381) (layer "B.Cu") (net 10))
 (segment (start 108.659212 54.02) (end 106.959212 55.72) (width 0.2032) (layer "B.Cu") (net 10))
 (segment (start 56.6 84.55) (end 58.65 86.6) (width 0.381) (layer "B.Cu") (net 10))
 (segment (start 81.1 84.25) (end 96.1 69.25) (width 0.381) (layer "B.Cu") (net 10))
 (segment (start 110.9975 76.54) (end 110.78 76.3225) (width 0.381) (layer "B.Cu") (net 10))
 (segment (start 108.4 52) (end 109 52.6) (width 0.381) (layer "B.Cu") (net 10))
 (segment (start 58.65 86.6) (end 81.1 86.6) (width 0.381) (layer "B.Cu") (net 10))
 (segment (start 99.7 56.87) (end 102.75 56.87) (width 0.381) (layer "B.Cu") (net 10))
 (segment (start 111.6 79.4) (end 110.9 78.7) (width 0.381) (layer "B.Cu") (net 10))
 (segment (start 117.3175 74.185) (end 114.9 76.6025) (width 0.381) (layer "B.Cu") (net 10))
 (segment (start 102.75 56.87) (end 105.98 60.1) (width 0.381) (layer "B.Cu") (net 10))
 (segment (start 109 52.6) (end 108.7375 52.8625) (width 0.381) (layer "B.Cu") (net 10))
 (segment (start 104.38 76.3575) (end 104.38 72.34) (width 0.381) (layer "B.Cu") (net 10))
 (segment (start 117.71 62.47) (end 113.45 62.47) (width 0.381) (layer "B.Cu") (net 10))
 (segment (start 113.45 62.47) (end 113.28 62.64) (width 0.381) (layer "B.Cu") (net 10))
 (segment (start 110.9975 78.6025) (end 110.9975 76.54) (width 0.381) (layer "B.Cu") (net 10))
 (segment (start 106.959212 55.72) (end 106.5375 55.72) (width 0.2032) (layer "B.Cu") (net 10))
 (segment (start 103.18 55.94) (end 101.84 55.94) (width 0.381) (layer "B.Cu") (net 10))
 (segment (start 100.9 52.5) (end 101.4 52) (width 0.381) (layer "B.Cu") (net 10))
 (segment (start 108.7375 54.02) (end 108.659212 54.02) (width 0.2032) (layer "B.Cu") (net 10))
 (segment (start 106.98 55.72) (end 106.5375 55.72) (width 0.381) (layer "B.Cu") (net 10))
 (segment (start 114.9 76.6025) (end 114.9 79.4) (width 0.381) (layer "B.Cu") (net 10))
 (segment (start 117.3175 73.6725) (end 117.3175 74.185) (width 0.381) (layer "B.Cu") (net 10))
 (segment (start 101.4 52) (end 108.4 52) (width 0.381) (layer "B.Cu") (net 10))
 (segment (start 81.1 86.6) (end 81.1 84.25) (width 0.381) (layer "B.Cu") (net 10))
 (segment (start 105.98 60.1) (end 105.98 60.94) (width 0.381) (layer "B.Cu") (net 10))
 (segment (start 114.9 79.4) (end 111.6 79.4) (width 0.381) (layer "B.Cu") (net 10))
 (segment (start 66.6 76.6) (end 95.8 76.6) (width 0.381) (layer "F.Cu") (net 8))
 (segment (start 62.7 72.7) (end 66.6 76.6) (width 0.381) (layer "F.Cu") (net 8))
 (via (at 62.7 72.7) (size 0.8) (drill 0.4) (layers "F.Cu" "B.Cu") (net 8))
 (via (at 95.8 76.6) (size 0.8) (drill 0.4) (layers "F.Cu" "B.Cu") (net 8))
 (segment (start 112.8975 76.54) (end 112.8975 73.6575) (width 0.381) (layer "B.Cu") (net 8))
 (segment (start 99.7 58.77) (end 103.78725 58.77) (width 0.381) (layer "B.Cu") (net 8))
 (segment (start 95.8 76.6) (end 95.84 76.64) (width 0.381) (layer "B.Cu") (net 8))
 (segment (start 112.8975 73.6575) (end 111.58 72.34) (width 0.381) (layer "B.Cu") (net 8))
 (segment (start 117.71 64.37) (end 116.78 63.44) (width 0.381) (layer "B.Cu") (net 8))
 (segment (start 61.1 66.3) (end 61.1 71.1) (width 0.381) (layer "B.Cu") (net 8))
 (segment (start 102.1975 73.7225) (end 103.58 72.34) (width 0.381) (layer "B.Cu") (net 8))
 (segment (start 105.18 60.16275) (end 105.18 60.94) (width 0.381) (layer "B.Cu") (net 8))
 (segment (start 95.84 76.64) (end 102.1975 76.64) (width 0.381) (layer "B.Cu") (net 8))
 (segment (start 103.78725 58.77) (end 105.18 60.16275) (width 0.381) (layer "B.Cu") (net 8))
 (segment (start 61.1 71.1) (end 62.7 72.7) (width 0.381) (layer "B.Cu") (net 8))
 (segment (start 116.78 63.44) (end 113.28 63.44) (width 0.381) (layer "B.Cu") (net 8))
 (segment (start 98.67 58.77) (end 99.7 58.77) (width 0.381) (layer "B.Cu") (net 8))
 (segment (start 96.12 57.0275) (end 96.9275 57.0275) (width 0.381) (layer "B.Cu") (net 8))
 (segment (start 96.9275 57.0275) (end 98.67 58.77) (width 0.381) (layer "B.Cu") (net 8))
 (segment (start 102.1975 76.64) (end 102.1975 73.7225) (width 0.381) (layer "B.Cu") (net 8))
 (segment (start 111.67 55.72) (end 111.84 55.89) (width 0.254) (layer "B.Cu") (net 16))
 (segment (start 107.58 56.8775) (end 107.58 60.94) (width 0.254) (layer "B.Cu") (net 16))
 (segment (start 108.7375 55.72) (end 111.67 55.72) (width 0.254) (layer "B.Cu") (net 16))
 (segment (start 108.7375 55.72) (end 107.58 56.8775) (width 0.254) (layer "B.Cu") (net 16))
 (segment (start 106.5375 54.02) (end 105.8375 54.02) (width 0.254) (layer "B.Cu") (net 11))
 (segment (start 105.8375 54.02) (end 105.2 54.6575) (width 0.254) (layer "B.Cu") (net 11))
 (segment (start 106.5175 54.04) (end 106.5375 54.02) (width 0.254) (layer "B.Cu") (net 11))
 (segment (start 105.2 54.6575) (end 105.2 57.228144) (width 0.254) (layer "B.Cu") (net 11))
 (segment (start 106.78 58.808144) (end 106.78 60.94) (width 0.254) (layer "B.Cu") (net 11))
 (segment (start 103.18 54.04) (end 106.5175 54.04) (width 0.254) (layer "B.Cu") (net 11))
 (segment (start 105.2 57.228144) (end 106.78 58.808144) (width 0.254) (layer "B.Cu") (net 11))
 (segment (start 138.1125 60.3875) (end 138.8334 61.1084) (width 0.254) (layer "B.Cu") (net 9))
 (segment (start 156.4416 61.1084) (end 157.1625 60.3875) (width 0.254) (layer "B.Cu") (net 9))
 (segment (start 138.8334 61.1084) (end 156.4416 61.1084) (width 0.254) (layer "B.Cu") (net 9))
 (segment (start 135.525 57.0875) (end 132.675 54.2375) (width 0.254) (layer "B.Cu") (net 2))
 (segment (start 138.1125 57.0875) (end 135.525 57.0875) (width 0.254) (layer "B.Cu") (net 2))
 (segment (start 154.575 57.0875) (end 151.725 54.2375) (width 0.254) (layer "B.Cu") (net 4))
 (segment (start 157.1625 57.0875) (end 154.575 57.0875) (width 0.254) (layer "B.Cu") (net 4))
 (segment (start 156.4416 80.1584) (end 138.8334 80.1584) (width 0.254) (layer "B.Cu") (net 17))
 (segment (start 157.1625 79.4375) (end 156.4416 80.1584) (width 0.254) (layer "B.Cu") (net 17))
 (segment (start 138.8334 80.1584) (end 138.1125 79.4375) (width 0.254) (layer "B.Cu") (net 17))
 (segment (start 135.525 76.1375) (end 132.675 73.2875) (width 0.254) (layer "B.Cu") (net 5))
 (segment (start 138.1125 76.1375) (end 135.525 76.1375) (width 0.254) (layer "B.Cu") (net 5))
 (segment (start 157.1625 76.1375) (end 154.575 76.1375) (width 0.254) (layer "B.Cu") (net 6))
 (segment (start 154.575 76.1375) (end 151.725 73.2875) (width 0.254) (layer "B.Cu") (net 6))
 (segment (start 66.41 57.29) (end 61.1 62.6) (width 0.254) (layer "B.Cu") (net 7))
 (segment (start 61.1 62.6) (end 61.1 63.5) (width 0.254) (layer "B.Cu") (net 7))
 (segment (start 66.41 55.24) (end 66.41 57.29) (width 0.254) (layer "B.Cu") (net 7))
 (segment (start 64.9 59.8) (end 64.8 59.9) (width 0.254) (layer "B.Cu") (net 48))
 (segment (start 64.9 63.3875) (end 67.5 65.9875) (width 0.254) (layer "B.Cu") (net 48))
 (segment (start 67.56 57.14) (end 64.9 59.8) (width 0.254) (layer "B.Cu") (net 48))
 (segment (start 64.9 59.8) (end 64.9 63.3875) (width 0.254) (layer "B.Cu") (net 48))
 (segment (start 67.56 55.24) (end 67.56 57.14) (width 0.254) (layer "B.Cu") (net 48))
 (segment (start 72.6 59.6875) (end 71.1875 61.1) (width 0.2) (layer "B.Cu") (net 47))
 (segment (start 68.56 58.4725) (end 71.1875 61.1) (width 0.2) (layer "B.Cu") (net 47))
 (segment (start 69.56 55.92033) (end 72.6 58.96033) (width 0.2) (layer "B.Cu") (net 47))
 (segment (start 68.56 55.24) (end 68.56 58.4725) (width 0.2) (layer "B.Cu") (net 47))
 (segment (start 69.56 55.24) (end 69.56 55.92033) (width 0.2) (layer "B.Cu") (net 47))
 (segment (start 72.6 58.96033) (end 72.6 59.6875) (width 0.2) (layer "B.Cu") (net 47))
 (segment (start 70.575213 57.924787) (end 67.7 60.8) (width 0.2) (layer "F.Cu") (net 13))
 (segment (start 67.7 60.8) (end 67.2 60.8) (width 0.2) (layer "F.Cu") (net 13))
 (via (at 70.575213 57.924787) (size 0.8) (drill 0.4) (layers "F.Cu" "B.Cu") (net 13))
 (segment (start 70.6 57.9) (end 70.575213 57.924787) (width 0.2) (layer "B.Cu") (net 13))
 (segment (start 68.06 55.24) (end 68.06 57.54) (width 0.2) (layer "B.Cu") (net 13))
 (segment (start 68.06 57.54) (end 66.9975 58.6025) (width 0.2) (layer "B.Cu") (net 13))
 (segment (start 68.06 60.0875) (end 67.91 60.2375) (width 0.2) (layer "B.Cu") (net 13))
 (segment (start 69.06 56.36) (end 70.6 57.9) (width 0.2) (layer "B.Cu") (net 13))
 (segment (start 66.9975 58.6025) (end 66.9975 61.15) (width 0.2) (layer "B.Cu") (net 13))
 (segment (start 69.06 55.24) (end 69.06 56.36) (width 0.2) (layer "B.Cu") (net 13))
 (segment (start 75.1 60.454582) (end 75.1 63.5875) (width 0.254) (layer "B.Cu") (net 15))
 (segment (start 70.56 55.24) (end 70.56 55.914582) (width 0.254) (layer "B.Cu") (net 15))
 (segment (start 70.56 55.914582) (end 75.1 60.454582) (width 0.254) (layer "B.Cu") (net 15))
 (segment (start 75.1 63.5875) (end 72.7 65.9875) (width 0.254) (layer "B.Cu") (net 15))
 (segment (start 126.365 56.1975) (end 126.365 75.2475) (width 0.254) (layer "F.Cu") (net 1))
 (segment (start 145.415 56.1975) (end 145.415 75.2475) (width 0.254) (layer "F.Cu") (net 3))
 (segment (start 114.4875 71.8475) (end 113.28 70.64) (width 0.254) (layer "B.Cu") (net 39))
 (segment (start 117.3175 71.8475) (end 114.4875 71.8475) (width 0.254) (layer "B.Cu") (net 39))
 (segment (start 73.5 71.2) (end 95.2 71.2) (width 0.254) (layer "F.Cu") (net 19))
 (segment (start 95.2 71.2) (end 95.3 71.2) (width 0.254) (layer "F.Cu") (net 19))
 (via (at 95.3 71.2) (size 0.8) (drill 0.4) (layers "F.Cu" "B.Cu") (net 19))
 (via (at 73.5 71.2) (size 0.8) (drill 0.4) (layers "F.Cu" "B.Cu") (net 19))
 (segment (start 70.6 65.4) (end 70.6 68.3) (width 0.254) (layer "B.Cu") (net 19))
 (segment (start 70.6 68.3) (end 73.5 71.2) (width 0.254) (layer "B.Cu") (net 19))
 (segment (start 95.3 71.2) (end 98.17 71.2) (width 0.254) (layer "B.Cu") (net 19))
 (segment (start 101.13 68.24) (end 101.88 68.24) (width 0.254) (layer "B.Cu") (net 19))
 (segment (start 73.0125 62.9875) (end 70.6 65.4) (width 0.254) (layer "B.Cu") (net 19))
 (segment (start 73.0125 61.1) (end 73.0125 62.9875) (width 0.254) (layer "B.Cu") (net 19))
 (segment (start 98.17 71.2) (end 101.13 68.24) (width 0.254) (layer "B.Cu") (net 19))
 (segment (start 73.1 72.3) (end 99.6 72.3) (width 0.254) (layer "F.Cu") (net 14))
 (via (at 99.6 72.3) (size 0.8) (drill 0.4) (layers "F.Cu" "B.Cu") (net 14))
 (via (at 73.1 72.3) (size 0.8) (drill 0.4) (layers "F.Cu" "B.Cu") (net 14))
 (segment (start 99.6 70.57) (end 101.13 69.04) (width 0.254) (layer "B.Cu") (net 14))
 (segment (start 68.8225 68.0225) (end 73.1 72.3) (width 0.254) (layer "B.Cu") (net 14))
 (segment (start 101.13 69.04) (end 101.88 69.04) (width 0.254) (layer "B.Cu") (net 14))
 (segment (start 68.8225 61.15) (end 68.8225 68.0225) (width 0.254) (layer "B.Cu") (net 14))
 (segment (start 99.6 72.3) (end 99.6 70.57) (width 0.254) (layer "B.Cu") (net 14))
 (segment (start 97.0675 59.8) (end 103.99 59.8) (width 0.254) (layer "B.Cu") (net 12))
 (segment (start 103.99 59.8) (end 104.38 60.19) (width 0.254) (layer "B.Cu") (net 12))
 (segment (start 104.38 60.19) (end 104.38 60.94) (width 0.254) (layer "B.Cu") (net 12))
 (segment (start 74.1225 80.85) (end 96.12 58.8525) (width 0.254) (layer "B.Cu") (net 12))
 (segment (start 62.8 80.85) (end 74.1225 80.85) (width 0.254) (layer "B.Cu") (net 12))
 (segment (start 96.12 58.8525) (end 97.0675 59.8) (width 0.254) (layer "B.Cu") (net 12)))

